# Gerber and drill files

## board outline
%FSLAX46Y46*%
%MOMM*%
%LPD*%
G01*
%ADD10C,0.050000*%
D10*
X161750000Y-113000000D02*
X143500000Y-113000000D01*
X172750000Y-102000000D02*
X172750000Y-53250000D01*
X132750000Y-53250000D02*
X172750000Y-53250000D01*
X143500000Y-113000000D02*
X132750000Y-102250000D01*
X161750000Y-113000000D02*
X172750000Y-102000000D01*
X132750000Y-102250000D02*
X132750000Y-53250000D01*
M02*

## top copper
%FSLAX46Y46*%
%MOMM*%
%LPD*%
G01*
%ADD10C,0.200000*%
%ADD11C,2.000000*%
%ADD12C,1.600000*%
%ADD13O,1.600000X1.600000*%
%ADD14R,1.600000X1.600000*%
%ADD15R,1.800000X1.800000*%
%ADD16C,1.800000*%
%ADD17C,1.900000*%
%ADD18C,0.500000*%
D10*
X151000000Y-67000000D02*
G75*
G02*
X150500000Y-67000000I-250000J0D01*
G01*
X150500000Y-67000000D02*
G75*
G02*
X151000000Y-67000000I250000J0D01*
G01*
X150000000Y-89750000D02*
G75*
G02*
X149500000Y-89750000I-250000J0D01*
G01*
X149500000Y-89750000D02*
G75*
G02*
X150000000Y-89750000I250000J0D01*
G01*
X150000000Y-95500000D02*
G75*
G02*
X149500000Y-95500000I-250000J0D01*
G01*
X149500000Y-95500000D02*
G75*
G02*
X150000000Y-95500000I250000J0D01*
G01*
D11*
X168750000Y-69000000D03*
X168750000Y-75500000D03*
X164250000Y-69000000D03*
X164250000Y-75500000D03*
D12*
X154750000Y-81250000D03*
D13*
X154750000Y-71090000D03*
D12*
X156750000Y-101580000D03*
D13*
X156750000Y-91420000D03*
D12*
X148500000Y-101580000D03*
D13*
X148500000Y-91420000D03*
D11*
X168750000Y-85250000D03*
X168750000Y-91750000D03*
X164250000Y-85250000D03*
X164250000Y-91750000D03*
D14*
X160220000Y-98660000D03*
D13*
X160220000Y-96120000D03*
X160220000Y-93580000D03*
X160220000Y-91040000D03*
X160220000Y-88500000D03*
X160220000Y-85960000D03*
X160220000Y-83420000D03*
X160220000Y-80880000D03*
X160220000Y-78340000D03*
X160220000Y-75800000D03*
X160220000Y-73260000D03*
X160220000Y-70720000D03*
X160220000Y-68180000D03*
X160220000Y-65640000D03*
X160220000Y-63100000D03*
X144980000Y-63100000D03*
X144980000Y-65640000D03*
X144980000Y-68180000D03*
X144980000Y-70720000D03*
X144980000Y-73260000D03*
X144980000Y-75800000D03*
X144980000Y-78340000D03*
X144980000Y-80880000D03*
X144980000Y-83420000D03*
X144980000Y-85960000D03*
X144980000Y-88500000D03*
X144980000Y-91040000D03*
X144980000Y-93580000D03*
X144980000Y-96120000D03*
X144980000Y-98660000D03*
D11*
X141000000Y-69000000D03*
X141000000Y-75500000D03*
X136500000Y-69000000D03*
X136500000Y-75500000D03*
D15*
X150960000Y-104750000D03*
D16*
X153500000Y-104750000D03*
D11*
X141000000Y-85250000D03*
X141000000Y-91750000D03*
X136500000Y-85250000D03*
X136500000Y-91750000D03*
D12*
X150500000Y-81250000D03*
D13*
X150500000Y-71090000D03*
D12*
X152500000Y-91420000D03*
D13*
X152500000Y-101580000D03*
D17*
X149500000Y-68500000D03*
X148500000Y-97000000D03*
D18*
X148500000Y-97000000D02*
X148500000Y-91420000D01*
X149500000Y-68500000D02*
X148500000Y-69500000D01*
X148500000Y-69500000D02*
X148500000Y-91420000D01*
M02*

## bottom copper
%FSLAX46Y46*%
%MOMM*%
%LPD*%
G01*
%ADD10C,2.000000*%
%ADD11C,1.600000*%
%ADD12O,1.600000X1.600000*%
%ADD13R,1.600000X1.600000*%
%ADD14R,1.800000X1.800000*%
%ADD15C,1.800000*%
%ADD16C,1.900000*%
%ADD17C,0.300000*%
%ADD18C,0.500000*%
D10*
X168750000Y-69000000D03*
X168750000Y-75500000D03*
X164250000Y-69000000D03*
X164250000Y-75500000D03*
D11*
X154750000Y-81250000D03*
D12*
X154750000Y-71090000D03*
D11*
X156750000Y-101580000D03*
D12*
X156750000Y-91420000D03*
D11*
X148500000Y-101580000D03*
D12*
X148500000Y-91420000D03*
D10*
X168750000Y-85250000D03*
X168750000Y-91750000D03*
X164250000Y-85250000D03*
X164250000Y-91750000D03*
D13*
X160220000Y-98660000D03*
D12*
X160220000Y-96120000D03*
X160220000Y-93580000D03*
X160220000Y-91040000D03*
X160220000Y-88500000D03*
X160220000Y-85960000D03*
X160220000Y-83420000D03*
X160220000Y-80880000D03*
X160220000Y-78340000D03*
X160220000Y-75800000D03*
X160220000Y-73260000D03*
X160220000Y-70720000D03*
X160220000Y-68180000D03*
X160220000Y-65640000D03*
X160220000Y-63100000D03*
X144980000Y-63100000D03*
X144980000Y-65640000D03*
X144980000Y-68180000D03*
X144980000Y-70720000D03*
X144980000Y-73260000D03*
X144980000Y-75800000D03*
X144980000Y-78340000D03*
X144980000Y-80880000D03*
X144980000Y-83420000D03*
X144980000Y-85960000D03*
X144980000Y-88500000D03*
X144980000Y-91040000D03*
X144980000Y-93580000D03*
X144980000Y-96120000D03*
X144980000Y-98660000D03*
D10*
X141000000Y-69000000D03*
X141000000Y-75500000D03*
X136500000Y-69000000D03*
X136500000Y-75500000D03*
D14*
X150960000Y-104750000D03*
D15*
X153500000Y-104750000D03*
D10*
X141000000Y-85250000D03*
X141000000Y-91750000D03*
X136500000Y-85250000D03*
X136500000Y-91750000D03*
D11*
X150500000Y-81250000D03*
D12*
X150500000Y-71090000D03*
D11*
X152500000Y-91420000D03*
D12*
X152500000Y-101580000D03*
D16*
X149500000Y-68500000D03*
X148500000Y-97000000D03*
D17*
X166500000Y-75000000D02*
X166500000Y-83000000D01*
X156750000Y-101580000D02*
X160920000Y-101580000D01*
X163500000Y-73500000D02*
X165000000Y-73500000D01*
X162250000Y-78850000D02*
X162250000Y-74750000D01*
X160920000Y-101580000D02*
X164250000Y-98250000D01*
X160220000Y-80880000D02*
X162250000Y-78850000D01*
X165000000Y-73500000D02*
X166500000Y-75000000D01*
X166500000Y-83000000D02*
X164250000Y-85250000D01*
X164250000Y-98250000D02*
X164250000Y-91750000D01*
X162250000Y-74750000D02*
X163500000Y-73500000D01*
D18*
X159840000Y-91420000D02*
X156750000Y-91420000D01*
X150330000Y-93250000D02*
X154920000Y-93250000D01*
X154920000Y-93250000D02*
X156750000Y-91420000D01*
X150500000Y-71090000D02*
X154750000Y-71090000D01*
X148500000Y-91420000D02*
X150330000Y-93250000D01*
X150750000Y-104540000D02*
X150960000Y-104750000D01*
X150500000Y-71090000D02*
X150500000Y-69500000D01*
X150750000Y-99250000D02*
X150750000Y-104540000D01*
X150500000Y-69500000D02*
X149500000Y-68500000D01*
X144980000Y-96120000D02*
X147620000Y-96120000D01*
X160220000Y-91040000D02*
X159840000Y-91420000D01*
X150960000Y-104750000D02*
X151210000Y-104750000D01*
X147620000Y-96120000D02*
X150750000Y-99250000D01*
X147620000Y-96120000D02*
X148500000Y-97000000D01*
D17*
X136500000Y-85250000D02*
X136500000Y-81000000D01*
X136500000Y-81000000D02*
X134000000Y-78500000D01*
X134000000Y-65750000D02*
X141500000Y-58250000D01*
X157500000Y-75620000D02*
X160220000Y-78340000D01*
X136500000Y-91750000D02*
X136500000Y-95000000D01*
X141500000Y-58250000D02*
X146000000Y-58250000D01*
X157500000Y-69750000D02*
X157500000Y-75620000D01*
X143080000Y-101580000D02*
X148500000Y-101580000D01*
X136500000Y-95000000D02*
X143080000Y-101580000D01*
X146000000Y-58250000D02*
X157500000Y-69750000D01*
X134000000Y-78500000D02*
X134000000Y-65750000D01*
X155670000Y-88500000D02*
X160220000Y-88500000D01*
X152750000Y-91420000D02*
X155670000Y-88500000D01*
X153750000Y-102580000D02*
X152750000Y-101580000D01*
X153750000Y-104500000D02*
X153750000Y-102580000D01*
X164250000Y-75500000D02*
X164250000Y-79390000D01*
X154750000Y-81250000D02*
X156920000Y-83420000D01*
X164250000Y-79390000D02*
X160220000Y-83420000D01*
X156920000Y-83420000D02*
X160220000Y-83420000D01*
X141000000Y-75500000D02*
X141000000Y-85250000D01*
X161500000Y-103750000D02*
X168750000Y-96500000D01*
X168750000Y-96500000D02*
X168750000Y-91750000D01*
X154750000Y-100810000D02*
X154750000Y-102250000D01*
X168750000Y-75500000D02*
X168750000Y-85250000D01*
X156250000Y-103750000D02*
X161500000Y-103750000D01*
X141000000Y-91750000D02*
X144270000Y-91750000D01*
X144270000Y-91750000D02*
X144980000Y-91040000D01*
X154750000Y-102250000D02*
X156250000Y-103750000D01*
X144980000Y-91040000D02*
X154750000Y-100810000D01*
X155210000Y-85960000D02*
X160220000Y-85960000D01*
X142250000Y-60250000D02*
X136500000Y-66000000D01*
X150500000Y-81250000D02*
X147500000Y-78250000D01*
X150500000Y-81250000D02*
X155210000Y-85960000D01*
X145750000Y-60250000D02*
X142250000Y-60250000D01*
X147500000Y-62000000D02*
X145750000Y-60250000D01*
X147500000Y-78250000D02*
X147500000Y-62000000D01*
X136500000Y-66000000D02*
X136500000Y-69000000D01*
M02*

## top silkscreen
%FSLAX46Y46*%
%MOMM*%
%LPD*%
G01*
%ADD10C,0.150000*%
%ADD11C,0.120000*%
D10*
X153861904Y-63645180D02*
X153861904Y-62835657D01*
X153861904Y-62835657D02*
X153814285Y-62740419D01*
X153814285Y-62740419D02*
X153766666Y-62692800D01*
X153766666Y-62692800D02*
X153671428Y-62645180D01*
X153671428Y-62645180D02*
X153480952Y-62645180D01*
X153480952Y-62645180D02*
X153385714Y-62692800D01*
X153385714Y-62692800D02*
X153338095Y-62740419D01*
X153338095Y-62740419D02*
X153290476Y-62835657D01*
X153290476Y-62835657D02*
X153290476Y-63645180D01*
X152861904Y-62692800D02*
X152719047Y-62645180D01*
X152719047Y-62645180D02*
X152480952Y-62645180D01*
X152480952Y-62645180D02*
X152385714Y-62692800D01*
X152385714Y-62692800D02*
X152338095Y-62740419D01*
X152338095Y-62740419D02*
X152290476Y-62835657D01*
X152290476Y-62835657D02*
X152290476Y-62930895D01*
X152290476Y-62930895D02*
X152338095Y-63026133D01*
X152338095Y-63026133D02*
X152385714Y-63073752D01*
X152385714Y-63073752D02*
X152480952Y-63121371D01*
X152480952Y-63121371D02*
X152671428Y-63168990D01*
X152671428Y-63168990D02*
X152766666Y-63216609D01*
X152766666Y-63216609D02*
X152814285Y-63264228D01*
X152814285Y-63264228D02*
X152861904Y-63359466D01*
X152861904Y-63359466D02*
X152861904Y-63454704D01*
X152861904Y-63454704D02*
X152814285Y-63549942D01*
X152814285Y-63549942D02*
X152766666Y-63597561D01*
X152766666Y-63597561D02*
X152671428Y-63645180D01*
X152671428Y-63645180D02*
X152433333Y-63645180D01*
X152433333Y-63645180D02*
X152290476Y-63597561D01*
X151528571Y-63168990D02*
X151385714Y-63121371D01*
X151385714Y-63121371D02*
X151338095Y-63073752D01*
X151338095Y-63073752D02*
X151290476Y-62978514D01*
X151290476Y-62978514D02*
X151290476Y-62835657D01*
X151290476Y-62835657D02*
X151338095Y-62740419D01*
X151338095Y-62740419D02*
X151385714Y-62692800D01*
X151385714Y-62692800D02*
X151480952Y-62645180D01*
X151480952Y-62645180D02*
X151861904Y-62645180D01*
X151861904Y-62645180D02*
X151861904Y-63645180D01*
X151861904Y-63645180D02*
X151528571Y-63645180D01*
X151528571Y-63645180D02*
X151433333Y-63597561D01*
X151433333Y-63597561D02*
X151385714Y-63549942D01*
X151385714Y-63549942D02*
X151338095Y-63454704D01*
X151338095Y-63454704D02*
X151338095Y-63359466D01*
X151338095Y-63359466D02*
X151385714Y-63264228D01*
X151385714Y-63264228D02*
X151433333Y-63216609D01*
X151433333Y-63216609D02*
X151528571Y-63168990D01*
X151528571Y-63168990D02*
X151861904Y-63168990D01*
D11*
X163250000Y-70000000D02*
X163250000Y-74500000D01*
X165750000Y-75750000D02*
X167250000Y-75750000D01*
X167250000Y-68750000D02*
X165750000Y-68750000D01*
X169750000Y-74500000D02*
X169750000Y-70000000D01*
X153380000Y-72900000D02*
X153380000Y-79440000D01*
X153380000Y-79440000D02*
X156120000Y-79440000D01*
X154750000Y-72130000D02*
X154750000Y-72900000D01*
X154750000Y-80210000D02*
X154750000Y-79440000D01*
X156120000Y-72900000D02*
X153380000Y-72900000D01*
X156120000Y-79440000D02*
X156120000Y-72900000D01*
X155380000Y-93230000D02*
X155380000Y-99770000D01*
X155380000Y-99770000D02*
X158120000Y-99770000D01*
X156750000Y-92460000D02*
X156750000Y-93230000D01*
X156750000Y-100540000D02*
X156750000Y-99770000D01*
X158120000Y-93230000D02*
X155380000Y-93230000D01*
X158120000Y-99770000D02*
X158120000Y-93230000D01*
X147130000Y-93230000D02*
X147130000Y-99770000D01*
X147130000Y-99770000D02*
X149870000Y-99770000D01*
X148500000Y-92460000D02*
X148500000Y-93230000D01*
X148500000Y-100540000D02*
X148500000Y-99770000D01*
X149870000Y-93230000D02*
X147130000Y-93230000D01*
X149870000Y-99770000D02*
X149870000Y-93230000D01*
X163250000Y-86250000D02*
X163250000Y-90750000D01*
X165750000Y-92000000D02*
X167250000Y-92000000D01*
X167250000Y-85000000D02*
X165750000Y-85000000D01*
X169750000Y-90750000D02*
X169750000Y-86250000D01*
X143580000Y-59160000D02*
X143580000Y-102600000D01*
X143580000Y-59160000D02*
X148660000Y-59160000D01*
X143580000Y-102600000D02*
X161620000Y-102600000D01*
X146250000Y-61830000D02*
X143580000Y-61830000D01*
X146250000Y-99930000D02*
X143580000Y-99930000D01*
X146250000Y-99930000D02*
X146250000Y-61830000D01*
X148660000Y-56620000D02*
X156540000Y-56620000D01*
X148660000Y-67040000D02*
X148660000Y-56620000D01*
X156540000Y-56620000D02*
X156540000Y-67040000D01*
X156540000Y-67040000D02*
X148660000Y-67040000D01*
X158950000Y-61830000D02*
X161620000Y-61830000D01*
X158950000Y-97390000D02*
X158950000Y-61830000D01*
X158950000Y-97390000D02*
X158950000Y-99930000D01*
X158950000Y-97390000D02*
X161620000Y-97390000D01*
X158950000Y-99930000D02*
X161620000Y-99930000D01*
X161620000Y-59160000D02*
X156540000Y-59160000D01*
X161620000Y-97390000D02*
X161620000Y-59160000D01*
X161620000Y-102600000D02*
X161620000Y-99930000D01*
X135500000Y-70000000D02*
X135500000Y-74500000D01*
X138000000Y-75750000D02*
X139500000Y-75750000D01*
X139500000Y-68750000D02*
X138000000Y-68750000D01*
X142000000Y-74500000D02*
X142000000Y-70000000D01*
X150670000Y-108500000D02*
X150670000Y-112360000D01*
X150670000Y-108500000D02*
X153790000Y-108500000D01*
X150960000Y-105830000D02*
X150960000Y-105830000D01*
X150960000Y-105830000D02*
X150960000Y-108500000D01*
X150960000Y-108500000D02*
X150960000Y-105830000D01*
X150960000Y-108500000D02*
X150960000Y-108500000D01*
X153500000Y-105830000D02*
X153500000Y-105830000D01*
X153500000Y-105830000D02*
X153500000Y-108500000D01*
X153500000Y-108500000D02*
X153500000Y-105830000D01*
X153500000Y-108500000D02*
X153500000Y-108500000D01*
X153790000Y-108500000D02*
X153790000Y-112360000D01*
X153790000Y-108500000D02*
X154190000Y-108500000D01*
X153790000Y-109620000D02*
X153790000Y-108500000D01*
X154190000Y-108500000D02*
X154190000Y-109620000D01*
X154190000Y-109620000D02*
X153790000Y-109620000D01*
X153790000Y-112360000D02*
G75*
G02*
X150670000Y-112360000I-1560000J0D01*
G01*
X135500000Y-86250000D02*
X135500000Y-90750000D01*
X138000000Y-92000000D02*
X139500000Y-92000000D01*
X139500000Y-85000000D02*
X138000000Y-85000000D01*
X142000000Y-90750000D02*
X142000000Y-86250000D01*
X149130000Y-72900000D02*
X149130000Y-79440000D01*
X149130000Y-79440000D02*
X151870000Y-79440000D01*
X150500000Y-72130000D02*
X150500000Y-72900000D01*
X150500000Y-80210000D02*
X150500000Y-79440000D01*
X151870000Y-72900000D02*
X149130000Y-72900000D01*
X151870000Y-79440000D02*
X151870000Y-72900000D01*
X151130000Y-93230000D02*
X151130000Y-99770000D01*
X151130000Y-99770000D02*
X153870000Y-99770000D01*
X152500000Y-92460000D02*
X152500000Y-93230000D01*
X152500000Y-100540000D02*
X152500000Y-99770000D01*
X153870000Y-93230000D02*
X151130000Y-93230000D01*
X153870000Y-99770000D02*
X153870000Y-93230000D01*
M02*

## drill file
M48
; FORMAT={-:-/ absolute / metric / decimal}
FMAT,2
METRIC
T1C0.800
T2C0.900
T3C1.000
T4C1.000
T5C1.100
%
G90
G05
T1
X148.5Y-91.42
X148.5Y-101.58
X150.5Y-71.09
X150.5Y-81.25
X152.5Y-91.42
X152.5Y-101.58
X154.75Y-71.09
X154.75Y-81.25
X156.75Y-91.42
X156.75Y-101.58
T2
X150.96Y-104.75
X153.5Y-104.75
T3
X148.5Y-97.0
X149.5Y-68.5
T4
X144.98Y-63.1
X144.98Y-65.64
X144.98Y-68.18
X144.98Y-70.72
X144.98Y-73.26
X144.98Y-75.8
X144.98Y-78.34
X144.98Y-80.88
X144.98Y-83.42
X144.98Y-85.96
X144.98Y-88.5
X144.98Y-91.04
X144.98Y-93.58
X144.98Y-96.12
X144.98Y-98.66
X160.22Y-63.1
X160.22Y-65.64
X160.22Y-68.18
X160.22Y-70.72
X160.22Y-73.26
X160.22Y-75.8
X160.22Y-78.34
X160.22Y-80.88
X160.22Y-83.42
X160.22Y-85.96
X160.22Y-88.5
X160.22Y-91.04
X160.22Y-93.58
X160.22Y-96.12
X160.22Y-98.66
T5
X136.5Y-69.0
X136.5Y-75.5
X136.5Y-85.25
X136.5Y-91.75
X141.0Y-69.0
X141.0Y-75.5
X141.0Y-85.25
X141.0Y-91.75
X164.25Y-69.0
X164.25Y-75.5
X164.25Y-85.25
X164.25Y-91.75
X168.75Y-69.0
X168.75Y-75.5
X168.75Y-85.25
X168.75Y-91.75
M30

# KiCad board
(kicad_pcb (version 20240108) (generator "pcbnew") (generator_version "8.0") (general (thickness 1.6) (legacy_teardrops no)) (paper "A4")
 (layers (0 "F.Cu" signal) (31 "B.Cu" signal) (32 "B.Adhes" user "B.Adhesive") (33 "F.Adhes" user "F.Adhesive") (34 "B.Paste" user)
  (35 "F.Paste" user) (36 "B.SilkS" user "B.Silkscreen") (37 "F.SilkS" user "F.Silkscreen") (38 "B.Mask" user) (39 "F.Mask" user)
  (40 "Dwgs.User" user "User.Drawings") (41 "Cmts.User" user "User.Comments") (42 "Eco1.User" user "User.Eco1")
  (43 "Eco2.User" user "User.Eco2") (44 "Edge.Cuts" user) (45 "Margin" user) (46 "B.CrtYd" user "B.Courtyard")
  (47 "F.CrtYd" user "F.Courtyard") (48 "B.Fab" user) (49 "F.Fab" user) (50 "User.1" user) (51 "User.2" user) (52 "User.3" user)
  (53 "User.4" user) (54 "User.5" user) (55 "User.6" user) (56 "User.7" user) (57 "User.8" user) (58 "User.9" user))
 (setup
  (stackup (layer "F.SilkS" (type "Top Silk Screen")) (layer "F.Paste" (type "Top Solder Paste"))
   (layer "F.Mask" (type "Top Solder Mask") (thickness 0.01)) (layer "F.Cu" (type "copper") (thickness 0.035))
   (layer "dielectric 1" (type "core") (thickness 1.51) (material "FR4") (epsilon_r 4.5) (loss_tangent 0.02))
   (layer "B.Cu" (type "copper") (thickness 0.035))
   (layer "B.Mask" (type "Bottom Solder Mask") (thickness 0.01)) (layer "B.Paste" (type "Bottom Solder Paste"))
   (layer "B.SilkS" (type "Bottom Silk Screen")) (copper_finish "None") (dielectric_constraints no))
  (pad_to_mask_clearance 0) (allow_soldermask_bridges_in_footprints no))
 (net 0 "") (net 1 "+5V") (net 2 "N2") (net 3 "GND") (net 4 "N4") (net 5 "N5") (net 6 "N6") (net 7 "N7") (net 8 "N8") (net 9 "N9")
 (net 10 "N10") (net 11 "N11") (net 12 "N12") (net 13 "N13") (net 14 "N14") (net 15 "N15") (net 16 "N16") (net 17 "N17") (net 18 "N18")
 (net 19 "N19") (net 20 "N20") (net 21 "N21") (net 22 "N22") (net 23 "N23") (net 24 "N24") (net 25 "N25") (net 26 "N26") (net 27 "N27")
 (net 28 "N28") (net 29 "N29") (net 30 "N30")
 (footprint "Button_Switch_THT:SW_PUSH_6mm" (layer "F.Cu") (at 168.75 69 -90)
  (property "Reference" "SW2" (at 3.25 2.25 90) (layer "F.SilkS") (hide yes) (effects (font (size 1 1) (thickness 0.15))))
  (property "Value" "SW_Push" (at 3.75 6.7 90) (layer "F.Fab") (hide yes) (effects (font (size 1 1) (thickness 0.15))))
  (fp_line (start 1 5.5) (end 5.5 5.5) (stroke (width 0.12) (type solid)) (layer "F.SilkS"))
  (fp_line (start 6.75 3) (end 6.75 1.5) (stroke (width 0.12) (type solid)) (layer "F.SilkS"))
  (fp_line (start -0.25 1.5) (end -0.25 3) (stroke (width 0.12) (type solid)) (layer "F.SilkS"))
  (fp_line (start 5.5 -1) (end 1 -1) (stroke (width 0.12) (type solid)) (layer "F.SilkS"))
  (pad "1" thru_hole circle (at 0 0) (size 2 2) (drill 1.1) (layers "*.Cu" "*.Mask") (remove_unused_layers no) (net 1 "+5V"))
  (pad "1" thru_hole circle (at 6.5 0) (size 2 2) (drill 1.1) (layers "*.Cu" "*.Mask") (remove_unused_layers no) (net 1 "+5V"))
  (pad "2" thru_hole circle (at 0 4.5) (size 2 2) (drill 1.1) (layers "*.Cu" "*.Mask") (remove_unused_layers no) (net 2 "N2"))
  (pad "2" thru_hole circle (at 6.5 4.5) (size 2 2) (drill 1.1) (layers "*.Cu" "*.Mask") (remove_unused_layers no) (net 2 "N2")))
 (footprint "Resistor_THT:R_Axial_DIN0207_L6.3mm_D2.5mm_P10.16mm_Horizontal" (layer "F.Cu") (at 154.75 81.25 90)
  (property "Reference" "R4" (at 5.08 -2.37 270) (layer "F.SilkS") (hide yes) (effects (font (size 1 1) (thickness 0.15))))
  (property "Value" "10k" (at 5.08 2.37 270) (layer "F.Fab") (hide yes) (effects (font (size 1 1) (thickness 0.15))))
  (fp_line (start 8.35 -1.37) (end 1.81 -1.37) (stroke (width 0.12) (type solid)) (layer "F.SilkS"))
  (fp_line (start 1.81 -1.37) (end 1.81 1.37) (stroke (width 0.12) (type solid)) (layer "F.SilkS"))
  (fp_line (start 9.12 0) (end 8.35 0) (stroke (width 0.12) (type solid)) (layer "F.SilkS"))
  (fp_line (start 1.04 0) (end 1.81 0) (stroke (width 0.12) (type solid)) (layer "F.SilkS"))
  (fp_line (start 8.35 1.37) (end 8.35 -1.37) (stroke (width 0.12) (type solid)) (layer "F.SilkS"))
  (fp_line (start 1.81 1.37) (end 8.35 1.37) (stroke (width 0.12) (type solid)) (layer "F.SilkS"))
  (pad "1" thru_hole circle (at 0 0 90) (size 1.6 1.6) (drill 0.8) (layers "*.Cu" "*.Mask") (remove_unused_layers no) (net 2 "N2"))
  (pad "2" thru_hole oval (at 10.16 0 90) (size 1.6 1.6) (drill 0.8) (layers "*.Cu" "*.Mask") (remove_unused_layers no) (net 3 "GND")))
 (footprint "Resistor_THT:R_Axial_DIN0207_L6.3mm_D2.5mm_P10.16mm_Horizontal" (layer "F.Cu") (at 156.75 101.58 90)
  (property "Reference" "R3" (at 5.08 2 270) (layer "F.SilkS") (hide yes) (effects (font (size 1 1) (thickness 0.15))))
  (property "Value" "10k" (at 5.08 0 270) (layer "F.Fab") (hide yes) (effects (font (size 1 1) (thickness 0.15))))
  (fp_line (start 8.35 -1.37) (end 1.81 -1.37) (stroke (width 0.12) (type solid)) (layer "F.SilkS"))
  (fp_line (start 1.81 -1.37) (end 1.81 1.37) (stroke (width 0.12) (type solid)) (layer "F.SilkS"))
  (fp_line (start 9.12 0) (end 8.35 0) (stroke (width 0.12) (type solid)) (layer "F.SilkS"))
  (fp_line (start 1.04 0) (end 1.81 0) (stroke (width 0.12) (type solid)) (layer "F.SilkS"))
  (fp_line (start 8.35 1.37) (end 8.35 -1.37) (stroke (width 0.12) (type solid)) (layer "F.SilkS"))
  (fp_line (start 1.81 1.37) (end 8.35 1.37) (stroke (width 0.12) (type solid)) (layer "F.SilkS"))
  (pad "1" thru_hole circle (at 0 0 90) (size 1.6 1.6) (drill 0.8) (layers "*.Cu" "*.Mask") (remove_unused_layers no) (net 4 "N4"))
  (pad "2" thru_hole oval (at 10.16 0 90) (size 1.6 1.6) (drill 0.8) (layers "*.Cu" "*.Mask") (remove_unused_layers no) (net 3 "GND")))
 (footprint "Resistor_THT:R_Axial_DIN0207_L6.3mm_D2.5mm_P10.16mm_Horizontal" (layer "F.Cu") (at 148.5 101.58 90)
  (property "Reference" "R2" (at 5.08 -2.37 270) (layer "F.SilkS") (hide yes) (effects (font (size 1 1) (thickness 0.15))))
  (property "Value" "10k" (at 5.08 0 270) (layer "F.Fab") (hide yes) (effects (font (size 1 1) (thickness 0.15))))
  (fp_line (start 8.35 -1.37) (end 1.81 -1.37) (stroke (width 0.12) (type solid)) (layer "F.SilkS"))
  (fp_line (start 1.81 -1.37) (end 1.81 1.37) (stroke (width 0.12) (type solid)) (layer "F.SilkS"))
  (fp_line (start 9.12 0) (end 8.35 0) (stroke (width 0.12) (type solid)) (layer "F.SilkS"))
  (fp_line (start 1.04 0) (end 1.81 0) (stroke (width 0.12) (type solid)) (layer "F.SilkS"))
  (fp_line (start 8.35 1.37) (end 8.35 -1.37) (stroke (width 0.12) (type solid)) (layer "F.SilkS"))
  (fp_line (start 1.81 1.37) (end 8.35 1.37) (stroke (width 0.12) (type solid)) (layer "F.SilkS"))
  (pad "1" thru_hole circle (at 0 0 90) (size 1.6 1.6) (drill 0.8) (layers "*.Cu" "*.Mask") (remove_unused_layers no) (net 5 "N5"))
  (pad "2" thru_hole oval (at 10.16 0 90) (size 1.6 1.6) (drill 0.8) (layers "*.Cu" "*.Mask") (remove_unused_layers no) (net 3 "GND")))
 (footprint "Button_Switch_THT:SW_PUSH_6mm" (layer "F.Cu") (at 168.75 85.25 -90)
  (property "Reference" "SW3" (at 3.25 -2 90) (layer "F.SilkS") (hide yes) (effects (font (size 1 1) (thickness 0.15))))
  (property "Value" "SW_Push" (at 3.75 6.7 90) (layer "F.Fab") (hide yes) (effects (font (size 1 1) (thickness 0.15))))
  (fp_line (start 1 5.5) (end 5.5 5.5) (stroke (width 0.12) (type solid)) (layer "F.SilkS"))
  (fp_line (start 6.75 3) (end 6.75 1.5) (stroke (width 0.12) (type solid)) (layer "F.SilkS"))
  (fp_line (start -0.25 1.5) (end -0.25 3) (stroke (width 0.12) (type solid)) (layer "F.SilkS"))
  (fp_line (start 5.5 -1) (end 1 -1) (stroke (width 0.12) (type solid)) (layer "F.SilkS"))
  (pad "1" thru_hole circle (at 0 0) (size 2 2) (drill 1.1) (layers "*.Cu" "*.Mask") (remove_unused_layers no) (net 1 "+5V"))
  (pad "1" thru_hole circle (at 6.5 0) (size 2 2) (drill 1.1) (layers "*.Cu" "*.Mask") (remove_unused_layers no) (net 1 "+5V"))
  (pad "2" thru_hole circle (at 0 4.5) (size 2 2) (drill 1.1) (layers "*.Cu" "*.Mask") (remove_unused_layers no) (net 4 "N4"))
  (pad "2" thru_hole circle (at 6.5 4.5) (size 2 2) (drill 1.1) (layers "*.Cu" "*.Mask") (remove_unused_layers no) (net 4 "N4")))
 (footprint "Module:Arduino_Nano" (layer "F.Cu") (at 160.22 98.66 180)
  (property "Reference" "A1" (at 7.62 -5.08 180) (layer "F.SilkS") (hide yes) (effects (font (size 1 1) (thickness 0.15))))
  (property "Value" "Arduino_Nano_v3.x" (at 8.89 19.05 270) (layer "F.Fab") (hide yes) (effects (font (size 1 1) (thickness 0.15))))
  (fp_line (start 16.64 39.5) (end 16.64 -3.94) (stroke (width 0.12) (type solid)) (layer "F.SilkS"))
  (fp_line (start 16.64 39.5) (end 11.56 39.5) (stroke (width 0.12) (type solid)) (layer "F.SilkS"))
  (fp_line (start 16.64 -3.94) (end -1.4 -3.94) (stroke (width 0.12) (type solid)) (layer "F.SilkS"))
  (fp_line (start 13.97 36.83) (end 16.64 36.83) (stroke (width 0.12) (type solid)) (layer "F.SilkS"))
  (fp_line (start 13.97 -1.27) (end 16.64 -1.27) (stroke (width 0.12) (type solid)) (layer "F.SilkS"))
  (fp_line (start 13.97 -1.27) (end 13.97 36.83) (stroke (width 0.12) (type solid)) (layer "F.SilkS"))
  (fp_line (start 11.56 42.04) (end 3.68 42.04) (stroke (width 0.12) (type solid)) (layer "F.SilkS"))
  (fp_line (start 11.56 31.62) (end 11.56 42.04) (stroke (width 0.12) (type solid)) (layer "F.SilkS"))
  (fp_line (start 3.68 42.04) (end 3.68 31.62) (stroke (width 0.12) (type solid)) (layer "F.SilkS"))
  (fp_line (start 3.68 31.62) (end 11.56 31.62) (stroke (width 0.12) (type solid)) (layer "F.SilkS"))
  (fp_line (start 1.27 36.83) (end -1.4 36.83) (stroke (width 0.12) (type solid)) (layer "F.SilkS"))
  (fp_line (start 1.27 1.27) (end 1.27 36.83) (stroke (width 0.12) (type solid)) (layer "F.SilkS"))
  (fp_line (start 1.27 1.27) (end 1.27 -1.27) (stroke (width 0.12) (type solid)) (layer "F.SilkS"))
  (fp_line (start 1.27 1.27) (end -1.4 1.27) (stroke (width 0.12) (type solid)) (layer "F.SilkS"))
  (fp_line (start 1.27 -1.27) (end -1.4 -1.27) (stroke (width 0.12) (type solid)) (layer "F.SilkS"))
  (fp_line (start -1.4 39.5) (end 3.68 39.5) (stroke (width 0.12) (type solid)) (layer "F.SilkS"))
  (fp_line (start -1.4 1.27) (end -1.4 39.5) (stroke (width 0.12) (type solid)) (layer "F.SilkS"))
  (fp_line (start -1.4 -3.94) (end -1.4 -1.27) (stroke (width 0.12) (type solid)) (layer "F.SilkS"))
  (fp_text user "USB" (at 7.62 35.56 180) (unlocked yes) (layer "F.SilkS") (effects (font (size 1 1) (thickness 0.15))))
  (pad "1" thru_hole rect (at 0 0 180) (size 1.6 1.6) (drill 1) (layers "*.Cu" "*.Mask") (remove_unused_layers no) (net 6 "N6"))
  (pad "2" thru_hole oval (at 0 2.54 180) (size 1.6 1.6) (drill 1) (layers "*.Cu" "*.Mask") (remove_unused_layers no) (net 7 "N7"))
  (pad "3" thru_hole oval (at 0 5.08 180) (size 1.6 1.6) (drill 1) (layers "*.Cu" "*.Mask") (remove_unused_layers no) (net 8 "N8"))
  (pad "4" thru_hole oval (at 0 7.62 180) (size 1.6 1.6) (drill 1) (layers "*.Cu" "*.Mask") (remove_unused_layers no) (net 3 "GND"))
  (pad "5" thru_hole oval (at 0 10.16 180) (size 1.6 1.6) (drill 1) (layers "*.Cu" "*.Mask") (remove_unused_layers no) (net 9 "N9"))
  (pad "6" thru_hole oval (at 0 12.7 180) (size 1.6 1.6) (drill 1) (layers "*.Cu" "*.Mask") (remove_unused_layers no) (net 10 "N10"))
  (pad "7" thru_hole oval (at 0 15.24 180) (size 1.6 1.6) (drill 1) (layers "*.Cu" "*.Mask") (remove_unused_layers no) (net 2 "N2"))
  (pad "8" thru_hole oval (at 0 17.78 180) (size 1.6 1.6) (drill 1) (layers "*.Cu" "*.Mask") (remove_unused_layers no) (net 4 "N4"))
  (pad "9" thru_hole oval (at 0 20.32 180) (size 1.6 1.6) (drill 1) (layers "*.Cu" "*.Mask") (remove_unused_layers no) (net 5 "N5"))
  (pad "10" thru_hole oval (at 0 22.86 180) (size 1.6 1.6) (drill 1) (layers "*.Cu" "*.Mask") (remove_unused_layers no) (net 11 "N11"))
  (pad "11" thru_hole oval (at 0 25.4 180) (size 1.6 1.6) (drill 1) (layers "*.Cu" "*.Mask") (remove_unused_layers no) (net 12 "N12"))
  (pad "12" thru_hole oval (at 0 27.94 180) (size 1.6 1.6) (drill 1) (layers "*.Cu" "*.Mask") (remove_unused_layers no) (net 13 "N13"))
  (pad "13" thru_hole oval (at 0 30.48 180) (size 1.6 1.6) (drill 1) (layers "*.Cu" "*.Mask") (remove_unused_layers no) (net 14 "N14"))
  (pad "14" thru_hole oval (at 0 33.02 180) (size 1.6 1.6) (drill 1) (layers "*.Cu" "*.Mask") (remove_unused_layers no) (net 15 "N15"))
  (pad "15" thru_hole oval (at 0 35.56 180) (size 1.6 1.6) (drill 1) (layers "*.Cu" "*.Mask") (remove_unused_layers no) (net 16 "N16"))
  (pad "16" thru_hole oval (at 15.24 35.56 180) (size 1.6 1.6) (drill 1) (layers "*.Cu" "*.Mask") (remove_unused_layers no) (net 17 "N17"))
  (pad "17" thru_hole oval (at 15.24 33.02 180) (size 1.6 1.6) (drill 1) (layers "*.Cu" "*.Mask") (remove_unused_layers no) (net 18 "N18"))
  (pad "18" thru_hole oval (at 15.24 30.48 180) (size 1.6 1.6) (drill 1) (layers "*.Cu" "*.Mask") (remove_unused_layers no) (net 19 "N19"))
  (pad "19" thru_hole oval (at 15.24 27.94 180) (size 1.6 1.6) (drill 1) (layers "*.Cu" "*.Mask") (remove_unused_layers no) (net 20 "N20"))
  (pad "20" thru_hole oval (at 15.24 25.4 180) (size 1.6 1.6) (drill 1) (layers "*.Cu" "*.Mask") (remove_unused_layers no) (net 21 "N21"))
  (pad "21" thru_hole oval (at 15.24 22.86 180) (size 1.6 1.6) (drill 1) (layers "*.Cu" "*.Mask") (remove_unused_layers no) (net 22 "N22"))
  (pad "22" thru_hole oval (at 15.24 20.32 180) (size 1.6 1.6) (drill 1) (layers "*.Cu" "*.Mask") (remove_unused_layers no) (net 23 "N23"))
  (pad "23" thru_hole oval (at 15.24 17.78 180) (size 1.6 1.6) (drill 1) (layers "*.Cu" "*.Mask") (remove_unused_layers no) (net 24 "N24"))
  (pad "24" thru_hole oval (at 15.24 15.24 180) (size 1.6 1.6) (drill 1) (layers "*.Cu" "*.Mask") (remove_unused_layers no) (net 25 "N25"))
  (pad "25" thru_hole oval (at 15.24 12.7 180) (size 1.6 1.6) (drill 1) (layers "*.Cu" "*.Mask") (remove_unused_layers no) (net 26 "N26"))
  (pad "26" thru_hole oval (at 15.24 10.16 180) (size 1.6 1.6) (drill 1) (layers "*.Cu" "*.Mask") (remove_unused_layers no) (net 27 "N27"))
  (pad "27" thru_hole oval (at 15.24 7.62 180) (size 1.6 1.6) (drill 1) (layers "*.Cu" "*.Mask") (remove_unused_layers no) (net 1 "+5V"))
  (pad "28" thru_hole oval (at 15.24 5.08 180) (size 1.6 1.6) (drill 1) (layers "*.Cu" "*.Mask") (remove_unused_layers no) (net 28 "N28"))
  (pad "29" thru_hole oval (at 15.24 2.54 180) (size 1.6 1.6) (drill 1) (layers "*.Cu" "*.Mask") (remove_unused_layers no) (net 3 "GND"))
  (pad "30" thru_hole oval (at 15.24 0 180) (size 1.6 1.6) (drill 1) (layers "*.Cu" "*.Mask") (remove_unused_layers no) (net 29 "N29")))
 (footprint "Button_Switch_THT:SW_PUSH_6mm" (layer "F.Cu") (at 141 69 -90)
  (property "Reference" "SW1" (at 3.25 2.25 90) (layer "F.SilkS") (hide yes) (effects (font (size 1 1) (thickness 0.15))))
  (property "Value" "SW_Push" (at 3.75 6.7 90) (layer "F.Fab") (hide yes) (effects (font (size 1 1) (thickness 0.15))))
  (fp_line (start 1 5.5) (end 5.5 5.5) (stroke (width 0.12) (type solid)) (layer "F.SilkS"))
  (fp_line (start 6.75 3) (end 6.75 1.5) (stroke (width 0.12) (type solid)) (layer "F.SilkS"))
  (fp_line (start -0.25 1.5) (end -0.25 3) (stroke (width 0.12) (type solid)) (layer "F.SilkS"))
  (fp_line (start 5.5 -1) (end 1 -1) (stroke (width 0.12) (type solid)) (layer "F.SilkS"))
  (pad "1" thru_hole circle (at 0 0) (size 2 2) (drill 1.1) (layers "*.Cu" "*.Mask") (remove_unused_layers no) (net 1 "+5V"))
  (pad "1" thru_hole circle (at 6.5 0) (size 2 2) (drill 1.1) (layers "*.Cu" "*.Mask") (remove_unused_layers no) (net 1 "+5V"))
  (pad "2" thru_hole circle (at 0 4.5) (size 2 2) (drill 1.1) (layers "*.Cu" "*.Mask") (remove_unused_layers no) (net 10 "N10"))
  (pad "2" thru_hole circle (at 6.5 4.5) (size 2 2) (drill 1.1) (layers "*.Cu" "*.Mask") (remove_unused_layers no) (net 10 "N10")))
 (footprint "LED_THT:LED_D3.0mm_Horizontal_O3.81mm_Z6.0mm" (layer "F.Cu") (at 150.96 104.75)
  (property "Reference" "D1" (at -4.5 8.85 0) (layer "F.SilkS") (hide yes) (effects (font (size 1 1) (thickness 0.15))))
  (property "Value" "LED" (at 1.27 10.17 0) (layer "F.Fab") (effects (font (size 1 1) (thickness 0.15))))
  (fp_line (start -0.29 3.75) (end -0.29 7.61) (stroke (width 0.12) (type solid)) (layer "F.SilkS"))
  (fp_line (start -0.29 3.75) (end 2.83 3.75) (stroke (width 0.12) (type solid)) (layer "F.SilkS"))
  (fp_line (start 0 1.08) (end 0 1.08) (stroke (width 0.12) (type solid)) (layer "F.SilkS"))
  (fp_line (start 0 1.08) (end 0 3.75) (stroke (width 0.12) (type solid)) (layer "F.SilkS"))
  (fp_line (start 0 3.75) (end 0 1.08) (stroke (width 0.12) (type solid)) (layer "F.SilkS"))
  (fp_line (start 0 3.75) (end 0 3.75) (stroke (width 0.12) (type solid)) (layer "F.SilkS"))
  (fp_line (start 2.54 1.08) (end 2.54 1.08) (stroke (width 0.12) (type solid)) (layer "F.SilkS"))
  (fp_line (start 2.54 1.08) (end 2.54 3.75) (stroke (width 0.12) (type solid)) (layer "F.SilkS"))
  (fp_line (start 2.54 3.75) (end 2.54 1.08) (stroke (width 0.12) (type solid)) (layer "F.SilkS"))
  (fp_line (start 2.54 3.75) (end 2.54 3.75) (stroke (width 0.12) (type solid)) (layer "F.SilkS"))
  (fp_line (start 2.83 3.75) (end 2.83 7.61) (stroke (width 0.12) (type solid)) (layer "F.SilkS"))
  (fp_line (start 2.83 3.75) (end 3.23 3.75) (stroke (width 0.12) (type solid)) (layer "F.SilkS"))
  (fp_line (start 2.83 4.87) (end 2.83 3.75) (stroke (width 0.12) (type solid)) (layer "F.SilkS"))
  (fp_line (start 3.23 3.75) (end 3.23 4.87) (stroke (width 0.12) (type solid)) (layer "F.SilkS"))
  (fp_line (start 3.23 4.87) (end 2.83 4.87) (stroke (width 0.12) (type solid)) (layer "F.SilkS"))
  (fp_arc (start 2.83 7.61) (mid 1.27 9.17) (end -0.29 7.61) (stroke (width 0.12) (type solid)) (layer "F.SilkS"))
  (pad "1" thru_hole rect (at 0 0) (size 1.8 1.8) (drill 0.9) (layers "*.Cu" "*.Mask") (remove_unused_layers no) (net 3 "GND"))
  (pad "2" thru_hole circle (at 2.54 0) (size 1.8 1.8) (drill 0.9) (layers "*.Cu" "*.Mask") (remove_unused_layers no) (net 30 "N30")))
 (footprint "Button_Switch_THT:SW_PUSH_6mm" (layer "F.Cu") (at 141 85.25 -90)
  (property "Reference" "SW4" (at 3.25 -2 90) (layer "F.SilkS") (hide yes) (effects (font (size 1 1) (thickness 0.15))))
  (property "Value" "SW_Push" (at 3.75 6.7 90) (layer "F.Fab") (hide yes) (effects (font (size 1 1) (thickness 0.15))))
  (fp_line (start 1 5.5) (end 5.5 5.5) (stroke (width 0.12) (type solid)) (layer "F.SilkS"))
  (fp_line (start 6.75 3) (end 6.75 1.5) (stroke (width 0.12) (type solid)) (layer "F.SilkS"))
  (fp_line (start -0.25 1.5) (end -0.25 3) (stroke (width 0.12) (type solid)) (layer "F.SilkS"))
  (fp_line (start 5.5 -1) (end 1 -1) (stroke (width 0.12) (type solid)) (layer "F.SilkS"))
  (pad "1" thru_hole circle (at 0 0) (size 2 2) (drill 1.1) (layers "*.Cu" "*.Mask") (remove_unused_layers no) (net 1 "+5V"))
  (pad "1" thru_hole circle (at 6.5 0) (size 2 2) (drill 1.1) (layers "*.Cu" "*.Mask") (remove_unused_layers no) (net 1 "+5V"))
  (pad "2" thru_hole circle (at 0 4.5) (size 2 2) (drill 1.1) (layers "*.Cu" "*.Mask") (remove_unused_layers no) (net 5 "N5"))
  (pad "2" thru_hole circle (at 6.5 4.5) (size 2 2) (drill 1.1) (layers "*.Cu" "*.Mask") (remove_unused_layers no) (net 5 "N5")))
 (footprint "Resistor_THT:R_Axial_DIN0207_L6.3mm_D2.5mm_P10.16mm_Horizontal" (layer "F.Cu") (at 150.5 81.25 90)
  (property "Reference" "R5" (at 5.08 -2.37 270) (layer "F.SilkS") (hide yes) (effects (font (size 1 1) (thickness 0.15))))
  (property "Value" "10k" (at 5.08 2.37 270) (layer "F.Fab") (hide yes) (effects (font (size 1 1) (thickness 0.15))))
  (fp_line (start 8.35 -1.37) (end 1.81 -1.37) (stroke (width 0.12) (type solid)) (layer "F.SilkS"))
  (fp_line (start 1.81 -1.37) (end 1.81 1.37) (stroke (width 0.12) (type solid)) (layer "F.SilkS"))
  (fp_line (start 9.12 0) (end 8.35 0) (stroke (width 0.12) (type solid)) (layer "F.SilkS"))
  (fp_line (start 1.04 0) (end 1.81 0) (stroke (width 0.12) (type solid)) (layer "F.SilkS"))
  (fp_line (start 8.35 1.37) (end 8.35 -1.37) (stroke (width 0.12) (type solid)) (layer "F.SilkS"))
  (fp_line (start 1.81 1.37) (end 8.35 1.37) (stroke (width 0.12) (type solid)) (layer "F.SilkS"))
  (pad "1" thru_hole circle (at 0 0 90) (size 1.6 1.6) (drill 0.8) (layers "*.Cu" "*.Mask") (remove_unused_layers no) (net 10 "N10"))
  (pad "2" thru_hole oval (at 10.16 0 90) (size 1.6 1.6) (drill 0.8) (layers "*.Cu" "*.Mask") (remove_unused_layers no) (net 3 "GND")))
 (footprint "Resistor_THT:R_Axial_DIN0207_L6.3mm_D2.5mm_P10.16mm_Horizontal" (layer "F.Cu") (at 152.5 91.42 -90)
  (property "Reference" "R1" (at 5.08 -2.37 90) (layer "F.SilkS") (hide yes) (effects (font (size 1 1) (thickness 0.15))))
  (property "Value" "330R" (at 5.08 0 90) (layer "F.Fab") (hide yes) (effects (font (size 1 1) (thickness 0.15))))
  (fp_line (start 1.81 1.37) (end 8.35 1.37) (stroke (width 0.12) (type solid)) (layer "F.SilkS"))
  (fp_line (start 8.35 1.37) (end 8.35 -1.37) (stroke (width 0.12) (type solid)) (layer "F.SilkS"))
  (fp_line (start 1.04 0) (end 1.81 0) (stroke (width 0.12) (type solid)) (layer "F.SilkS"))
  (fp_line (start 9.12 0) (end 8.35 0) (stroke (width 0.12) (type solid)) (layer "F.SilkS"))
  (fp_line (start 1.81 -1.37) (end 1.81 1.37) (stroke (width 0.12) (type solid)) (layer "F.SilkS"))
  (fp_line (start 8.35 -1.37) (end 1.81 -1.37) (stroke (width 0.12) (type solid)) (layer "F.SilkS"))
  (pad "1" thru_hole circle (at 0 0 270) (size 1.6 1.6) (drill 0.8) (layers "*.Cu" "*.Mask") (remove_unused_layers no) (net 9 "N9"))
  (pad "2" thru_hole oval (at 10.16 0 270) (size 1.6 1.6) (drill 0.8) (layers "*.Cu" "*.Mask") (remove_unused_layers no) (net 30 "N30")))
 (gr_circle (center 150.75 67) (end 151 67) (stroke (width 0.2) (type default)) (fill none) (layer "F.Cu"))
 (gr_circle (center 149.75 89.75) (end 150 89.75) (stroke (width 0.2) (type default)) (fill none) (layer "F.Cu"))
 (gr_circle (center 149.75 95.5) (end 150 95.5) (stroke (width 0.2) (type default)) (fill none) (layer "F.Cu"))
 (gr_line (start 161.75 113) (end 143.5 113) (stroke (width 0.05) (type default)) (layer "Edge.Cuts"))
 (gr_line (start 172.75 102) (end 172.75 53.25) (stroke (width 0.05) (type default)) (layer "Edge.Cuts"))
 (gr_line (start 132.75 53.25) (end 172.75 53.25) (stroke (width 0.05) (type default)) (layer "Edge.Cuts"))
 (gr_line (start 143.5 113) (end 132.75 102.25) (stroke (width 0.05) (type default)) (layer "Edge.Cuts"))
 (gr_line (start 161.75 113) (end 172.75 102) (stroke (width 0.05) (type default)) (layer "Edge.Cuts"))
 (gr_line (start 132.75 102.25) (end 132.75 53.25) (stroke (width 0.05) (type default)) (layer "Edge.Cuts"))
 (segment (start 166.5 75) (end 166.5 83) (width 0.3) (layer "B.Cu") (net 4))
 (segment (start 156.75 101.58) (end 160.92 101.58) (width 0.3) (layer "B.Cu") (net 4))
 (segment (start 163.5 73.5) (end 165 73.5) (width 0.3) (layer "B.Cu") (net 4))
 (segment (start 162.25 78.85) (end 162.25 74.75) (width 0.3) (layer "B.Cu") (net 4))
 (segment (start 160.92 101.58) (end 164.25 98.25) (width 0.3) (layer "B.Cu") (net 4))
 (segment (start 160.22 80.88) (end 162.25 78.85) (width 0.3) (layer "B.Cu") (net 4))
 (segment (start 165 73.5) (end 166.5 75) (width 0.3) (layer "B.Cu") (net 4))
 (segment (start 166.5 83) (end 164.25 85.25) (width 0.3) (layer "B.Cu") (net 4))
 (segment (start 164.25 98.25) (end 164.25 91.75) (width 0.3) (layer "B.Cu") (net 4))
 (segment (start 162.25 74.75) (end 163.5 73.5) (width 0.3) (layer "B.Cu") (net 4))
 (segment (start 148.5 97) (end 148.5 91.42) (width 0.5) (layer "F.Cu") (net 3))
 (segment (start 149.5 68.5) (end 148.5 69.5) (width 0.5) (layer "F.Cu") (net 3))
 (segment (start 148.5 69.5) (end 148.5 91.42) (width 0.5) (layer "F.Cu") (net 3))
 (via (at 149.5 68.5) (size 1.9) (drill 1) (layers "F.Cu" "B.Cu") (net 3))
 (via (at 148.5 97) (size 1.9) (drill 1) (layers "F.Cu" "B.Cu") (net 3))
 (segment (start 159.84 91.42) (end 156.75 91.42) (width 0.5) (layer "B.Cu") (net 3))
 (segment (start 150.33 93.25) (end 154.92 93.25) (width 0.5) (layer "B.Cu") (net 3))
 (segment (start 154.92 93.25) (end 156.75 91.42) (width 0.5) (layer "B.Cu") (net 3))
 (segment (start 150.5 71.09) (end 154.75 71.09) (width 0.5) (layer "B.Cu") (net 3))
 (segment (start 148.5 91.42) (end 150.33 93.25) (width 0.5) (layer "B.Cu") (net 3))
 (segment (start 150.75 104.54) (end 150.96 104.75) (width 0.5) (layer "B.Cu") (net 3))
 (segment (start 150.5 71.09) (end 150.5 69.5) (width 0.5) (layer "B.Cu") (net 3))
 (segment (start 150.75 99.25) (end 150.75 104.54) (width 0.5) (layer "B.Cu") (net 3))
 (segment (start 150.5 69.5) (end 149.5 68.5) (width 0.5) (layer "B.Cu") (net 3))
 (segment (start 144.98 96.12) (end 147.62 96.12) (width 0.5) (layer "B.Cu") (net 3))
 (segment (start 160.22 91.04) (end 159.84 91.42) (width 0.5) (layer "B.Cu") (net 3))
 (segment (start 150.96 104.75) (end 151.21 104.75) (width 0.5) (layer "B.Cu") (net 3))
 (segment (start 147.62 96.12) (end 150.75 99.25) (width 0.5) (layer "B.Cu") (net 3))
 (segment (start 147.62 96.12) (end 148.5 97) (width 0.5) (layer "B.Cu") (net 3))
 (segment (start 136.5 85.25) (end 136.5 81) (width 0.3) (layer "B.Cu") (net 5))
 (segment (start 136.5 81) (end 134 78.5) (width 0.3) (layer "B.Cu") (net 5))
 (segment (start 134 65.75) (end 141.5 58.25) (width 0.3) (layer "B.Cu") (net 5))
 (segment (start 157.5 75.62) (end 160.22 78.34) (width 0.3) (layer "B.Cu") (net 5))
 (segment (start 136.5 91.75) (end 136.5 95) (width 0.3) (layer "B.Cu") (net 5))
 (segment (start 141.5 58.25) (end 146 58.25) (width 0.3) (layer "B.Cu") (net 5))
 (segment (start 157.5 69.75) (end 157.5 75.62) (width 0.3) (layer "B.Cu") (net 5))
 (segment (start 143.08 101.58) (end 148.5 101.58) (width 0.3) (layer "B.Cu") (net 5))
 (segment (start 136.5 95) (end 143.08 101.58) (width 0.3) (layer "B.Cu") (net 5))
 (segment (start 146 58.25) (end 157.5 69.75) (width 0.3) (layer "B.Cu") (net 5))
 (segment (start 134 78.5) (end 134 65.75) (width 0.3) (layer "B.Cu") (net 5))
 (segment (start 155.67 88.5) (end 160.22 88.5) (width 0.3) (layer "B.Cu") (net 9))
 (segment (start 152.75 91.42) (end 155.67 88.5) (width 0.3) (layer "B.Cu") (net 9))
 (segment (start 153.75 102.58) (end 152.75 101.58) (width 0.3) (layer "B.Cu") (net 30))
 (segment (start 153.75 104.5) (end 153.75 102.58) (width 0.3) (layer "B.Cu") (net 30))
 (segment (start 164.25 75.5) (end 164.25 79.39) (width 0.3) (layer "B.Cu") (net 2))
 (segment (start 154.75 81.25) (end 156.92 83.42) (width 0.3) (layer "B.Cu") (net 2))
 (segment (start 164.25 79.39) (end 160.22 83.42) (width 0.3) (layer "B.Cu") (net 2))
 (segment (start 156.92 83.42) (end 160.22 83.42) (width 0.3) (layer "B.Cu") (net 2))
 (segment (start 141 75.5) (end 141 85.25) (width 0.3) (layer "B.Cu") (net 1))
 (segment (start 161.5 103.75) (end 168.75 96.5) (width 0.3) (layer "B.Cu") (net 1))
 (segment (start 168.75 96.5) (end 168.75 91.75) (width 0.3) (layer "B.Cu") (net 1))
 (segment (start 154.75 100.81) (end 154.75 102.25) (width 0.3) (layer "B.Cu") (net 1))
 (segment (start 168.75 75.5) (end 168.75 85.25) (width 0.3) (layer "B.Cu") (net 1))
 (segment (start 156.25 103.75) (end 161.5 103.75) (width 0.3) (layer "B.Cu") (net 1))
 (segment (start 141 91.75) (end 144.27 91.75) (width 0.3) (layer "B.Cu") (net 1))
 (segment (start 144.27 91.75) (end 144.98 91.04) (width 0.3) (layer "B.Cu") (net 1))
 (segment (start 154.75 102.25) (end 156.25 103.75) (width 0.3) (layer "B.Cu") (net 1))
 (segment (start 144.98 91.04) (end 154.75 100.81) (width 0.3) (layer "B.Cu") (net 1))
 (segment (start 155.21 85.96) (end 160.22 85.96) (width 0.3) (layer "B.Cu") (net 10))
 (segment (start 142.25 60.25) (end 136.5 66) (width 0.3) (layer "B.Cu") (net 10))
 (segment (start 150.5 81.25) (end 147.5 78.25) (width 0.3) (layer "B.Cu") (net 10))
 (segment (start 150.5 81.25) (end 155.21 85.96) (width 0.3) (layer "B.Cu") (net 10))
 (segment (start 145.75 60.25) (end 142.25 60.25) (width 0.3) (layer "B.Cu") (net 10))
 (segment (start 147.5 62) (end 145.75 60.25) (width 0.3) (layer "B.Cu") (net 10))
 (segment (start 147.5 78.25) (end 147.5 62) (width 0.3) (layer "B.Cu") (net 10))
 (segment (start 136.5 66) (end 136.5 69) (width 0.3) (layer "B.Cu") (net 10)))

